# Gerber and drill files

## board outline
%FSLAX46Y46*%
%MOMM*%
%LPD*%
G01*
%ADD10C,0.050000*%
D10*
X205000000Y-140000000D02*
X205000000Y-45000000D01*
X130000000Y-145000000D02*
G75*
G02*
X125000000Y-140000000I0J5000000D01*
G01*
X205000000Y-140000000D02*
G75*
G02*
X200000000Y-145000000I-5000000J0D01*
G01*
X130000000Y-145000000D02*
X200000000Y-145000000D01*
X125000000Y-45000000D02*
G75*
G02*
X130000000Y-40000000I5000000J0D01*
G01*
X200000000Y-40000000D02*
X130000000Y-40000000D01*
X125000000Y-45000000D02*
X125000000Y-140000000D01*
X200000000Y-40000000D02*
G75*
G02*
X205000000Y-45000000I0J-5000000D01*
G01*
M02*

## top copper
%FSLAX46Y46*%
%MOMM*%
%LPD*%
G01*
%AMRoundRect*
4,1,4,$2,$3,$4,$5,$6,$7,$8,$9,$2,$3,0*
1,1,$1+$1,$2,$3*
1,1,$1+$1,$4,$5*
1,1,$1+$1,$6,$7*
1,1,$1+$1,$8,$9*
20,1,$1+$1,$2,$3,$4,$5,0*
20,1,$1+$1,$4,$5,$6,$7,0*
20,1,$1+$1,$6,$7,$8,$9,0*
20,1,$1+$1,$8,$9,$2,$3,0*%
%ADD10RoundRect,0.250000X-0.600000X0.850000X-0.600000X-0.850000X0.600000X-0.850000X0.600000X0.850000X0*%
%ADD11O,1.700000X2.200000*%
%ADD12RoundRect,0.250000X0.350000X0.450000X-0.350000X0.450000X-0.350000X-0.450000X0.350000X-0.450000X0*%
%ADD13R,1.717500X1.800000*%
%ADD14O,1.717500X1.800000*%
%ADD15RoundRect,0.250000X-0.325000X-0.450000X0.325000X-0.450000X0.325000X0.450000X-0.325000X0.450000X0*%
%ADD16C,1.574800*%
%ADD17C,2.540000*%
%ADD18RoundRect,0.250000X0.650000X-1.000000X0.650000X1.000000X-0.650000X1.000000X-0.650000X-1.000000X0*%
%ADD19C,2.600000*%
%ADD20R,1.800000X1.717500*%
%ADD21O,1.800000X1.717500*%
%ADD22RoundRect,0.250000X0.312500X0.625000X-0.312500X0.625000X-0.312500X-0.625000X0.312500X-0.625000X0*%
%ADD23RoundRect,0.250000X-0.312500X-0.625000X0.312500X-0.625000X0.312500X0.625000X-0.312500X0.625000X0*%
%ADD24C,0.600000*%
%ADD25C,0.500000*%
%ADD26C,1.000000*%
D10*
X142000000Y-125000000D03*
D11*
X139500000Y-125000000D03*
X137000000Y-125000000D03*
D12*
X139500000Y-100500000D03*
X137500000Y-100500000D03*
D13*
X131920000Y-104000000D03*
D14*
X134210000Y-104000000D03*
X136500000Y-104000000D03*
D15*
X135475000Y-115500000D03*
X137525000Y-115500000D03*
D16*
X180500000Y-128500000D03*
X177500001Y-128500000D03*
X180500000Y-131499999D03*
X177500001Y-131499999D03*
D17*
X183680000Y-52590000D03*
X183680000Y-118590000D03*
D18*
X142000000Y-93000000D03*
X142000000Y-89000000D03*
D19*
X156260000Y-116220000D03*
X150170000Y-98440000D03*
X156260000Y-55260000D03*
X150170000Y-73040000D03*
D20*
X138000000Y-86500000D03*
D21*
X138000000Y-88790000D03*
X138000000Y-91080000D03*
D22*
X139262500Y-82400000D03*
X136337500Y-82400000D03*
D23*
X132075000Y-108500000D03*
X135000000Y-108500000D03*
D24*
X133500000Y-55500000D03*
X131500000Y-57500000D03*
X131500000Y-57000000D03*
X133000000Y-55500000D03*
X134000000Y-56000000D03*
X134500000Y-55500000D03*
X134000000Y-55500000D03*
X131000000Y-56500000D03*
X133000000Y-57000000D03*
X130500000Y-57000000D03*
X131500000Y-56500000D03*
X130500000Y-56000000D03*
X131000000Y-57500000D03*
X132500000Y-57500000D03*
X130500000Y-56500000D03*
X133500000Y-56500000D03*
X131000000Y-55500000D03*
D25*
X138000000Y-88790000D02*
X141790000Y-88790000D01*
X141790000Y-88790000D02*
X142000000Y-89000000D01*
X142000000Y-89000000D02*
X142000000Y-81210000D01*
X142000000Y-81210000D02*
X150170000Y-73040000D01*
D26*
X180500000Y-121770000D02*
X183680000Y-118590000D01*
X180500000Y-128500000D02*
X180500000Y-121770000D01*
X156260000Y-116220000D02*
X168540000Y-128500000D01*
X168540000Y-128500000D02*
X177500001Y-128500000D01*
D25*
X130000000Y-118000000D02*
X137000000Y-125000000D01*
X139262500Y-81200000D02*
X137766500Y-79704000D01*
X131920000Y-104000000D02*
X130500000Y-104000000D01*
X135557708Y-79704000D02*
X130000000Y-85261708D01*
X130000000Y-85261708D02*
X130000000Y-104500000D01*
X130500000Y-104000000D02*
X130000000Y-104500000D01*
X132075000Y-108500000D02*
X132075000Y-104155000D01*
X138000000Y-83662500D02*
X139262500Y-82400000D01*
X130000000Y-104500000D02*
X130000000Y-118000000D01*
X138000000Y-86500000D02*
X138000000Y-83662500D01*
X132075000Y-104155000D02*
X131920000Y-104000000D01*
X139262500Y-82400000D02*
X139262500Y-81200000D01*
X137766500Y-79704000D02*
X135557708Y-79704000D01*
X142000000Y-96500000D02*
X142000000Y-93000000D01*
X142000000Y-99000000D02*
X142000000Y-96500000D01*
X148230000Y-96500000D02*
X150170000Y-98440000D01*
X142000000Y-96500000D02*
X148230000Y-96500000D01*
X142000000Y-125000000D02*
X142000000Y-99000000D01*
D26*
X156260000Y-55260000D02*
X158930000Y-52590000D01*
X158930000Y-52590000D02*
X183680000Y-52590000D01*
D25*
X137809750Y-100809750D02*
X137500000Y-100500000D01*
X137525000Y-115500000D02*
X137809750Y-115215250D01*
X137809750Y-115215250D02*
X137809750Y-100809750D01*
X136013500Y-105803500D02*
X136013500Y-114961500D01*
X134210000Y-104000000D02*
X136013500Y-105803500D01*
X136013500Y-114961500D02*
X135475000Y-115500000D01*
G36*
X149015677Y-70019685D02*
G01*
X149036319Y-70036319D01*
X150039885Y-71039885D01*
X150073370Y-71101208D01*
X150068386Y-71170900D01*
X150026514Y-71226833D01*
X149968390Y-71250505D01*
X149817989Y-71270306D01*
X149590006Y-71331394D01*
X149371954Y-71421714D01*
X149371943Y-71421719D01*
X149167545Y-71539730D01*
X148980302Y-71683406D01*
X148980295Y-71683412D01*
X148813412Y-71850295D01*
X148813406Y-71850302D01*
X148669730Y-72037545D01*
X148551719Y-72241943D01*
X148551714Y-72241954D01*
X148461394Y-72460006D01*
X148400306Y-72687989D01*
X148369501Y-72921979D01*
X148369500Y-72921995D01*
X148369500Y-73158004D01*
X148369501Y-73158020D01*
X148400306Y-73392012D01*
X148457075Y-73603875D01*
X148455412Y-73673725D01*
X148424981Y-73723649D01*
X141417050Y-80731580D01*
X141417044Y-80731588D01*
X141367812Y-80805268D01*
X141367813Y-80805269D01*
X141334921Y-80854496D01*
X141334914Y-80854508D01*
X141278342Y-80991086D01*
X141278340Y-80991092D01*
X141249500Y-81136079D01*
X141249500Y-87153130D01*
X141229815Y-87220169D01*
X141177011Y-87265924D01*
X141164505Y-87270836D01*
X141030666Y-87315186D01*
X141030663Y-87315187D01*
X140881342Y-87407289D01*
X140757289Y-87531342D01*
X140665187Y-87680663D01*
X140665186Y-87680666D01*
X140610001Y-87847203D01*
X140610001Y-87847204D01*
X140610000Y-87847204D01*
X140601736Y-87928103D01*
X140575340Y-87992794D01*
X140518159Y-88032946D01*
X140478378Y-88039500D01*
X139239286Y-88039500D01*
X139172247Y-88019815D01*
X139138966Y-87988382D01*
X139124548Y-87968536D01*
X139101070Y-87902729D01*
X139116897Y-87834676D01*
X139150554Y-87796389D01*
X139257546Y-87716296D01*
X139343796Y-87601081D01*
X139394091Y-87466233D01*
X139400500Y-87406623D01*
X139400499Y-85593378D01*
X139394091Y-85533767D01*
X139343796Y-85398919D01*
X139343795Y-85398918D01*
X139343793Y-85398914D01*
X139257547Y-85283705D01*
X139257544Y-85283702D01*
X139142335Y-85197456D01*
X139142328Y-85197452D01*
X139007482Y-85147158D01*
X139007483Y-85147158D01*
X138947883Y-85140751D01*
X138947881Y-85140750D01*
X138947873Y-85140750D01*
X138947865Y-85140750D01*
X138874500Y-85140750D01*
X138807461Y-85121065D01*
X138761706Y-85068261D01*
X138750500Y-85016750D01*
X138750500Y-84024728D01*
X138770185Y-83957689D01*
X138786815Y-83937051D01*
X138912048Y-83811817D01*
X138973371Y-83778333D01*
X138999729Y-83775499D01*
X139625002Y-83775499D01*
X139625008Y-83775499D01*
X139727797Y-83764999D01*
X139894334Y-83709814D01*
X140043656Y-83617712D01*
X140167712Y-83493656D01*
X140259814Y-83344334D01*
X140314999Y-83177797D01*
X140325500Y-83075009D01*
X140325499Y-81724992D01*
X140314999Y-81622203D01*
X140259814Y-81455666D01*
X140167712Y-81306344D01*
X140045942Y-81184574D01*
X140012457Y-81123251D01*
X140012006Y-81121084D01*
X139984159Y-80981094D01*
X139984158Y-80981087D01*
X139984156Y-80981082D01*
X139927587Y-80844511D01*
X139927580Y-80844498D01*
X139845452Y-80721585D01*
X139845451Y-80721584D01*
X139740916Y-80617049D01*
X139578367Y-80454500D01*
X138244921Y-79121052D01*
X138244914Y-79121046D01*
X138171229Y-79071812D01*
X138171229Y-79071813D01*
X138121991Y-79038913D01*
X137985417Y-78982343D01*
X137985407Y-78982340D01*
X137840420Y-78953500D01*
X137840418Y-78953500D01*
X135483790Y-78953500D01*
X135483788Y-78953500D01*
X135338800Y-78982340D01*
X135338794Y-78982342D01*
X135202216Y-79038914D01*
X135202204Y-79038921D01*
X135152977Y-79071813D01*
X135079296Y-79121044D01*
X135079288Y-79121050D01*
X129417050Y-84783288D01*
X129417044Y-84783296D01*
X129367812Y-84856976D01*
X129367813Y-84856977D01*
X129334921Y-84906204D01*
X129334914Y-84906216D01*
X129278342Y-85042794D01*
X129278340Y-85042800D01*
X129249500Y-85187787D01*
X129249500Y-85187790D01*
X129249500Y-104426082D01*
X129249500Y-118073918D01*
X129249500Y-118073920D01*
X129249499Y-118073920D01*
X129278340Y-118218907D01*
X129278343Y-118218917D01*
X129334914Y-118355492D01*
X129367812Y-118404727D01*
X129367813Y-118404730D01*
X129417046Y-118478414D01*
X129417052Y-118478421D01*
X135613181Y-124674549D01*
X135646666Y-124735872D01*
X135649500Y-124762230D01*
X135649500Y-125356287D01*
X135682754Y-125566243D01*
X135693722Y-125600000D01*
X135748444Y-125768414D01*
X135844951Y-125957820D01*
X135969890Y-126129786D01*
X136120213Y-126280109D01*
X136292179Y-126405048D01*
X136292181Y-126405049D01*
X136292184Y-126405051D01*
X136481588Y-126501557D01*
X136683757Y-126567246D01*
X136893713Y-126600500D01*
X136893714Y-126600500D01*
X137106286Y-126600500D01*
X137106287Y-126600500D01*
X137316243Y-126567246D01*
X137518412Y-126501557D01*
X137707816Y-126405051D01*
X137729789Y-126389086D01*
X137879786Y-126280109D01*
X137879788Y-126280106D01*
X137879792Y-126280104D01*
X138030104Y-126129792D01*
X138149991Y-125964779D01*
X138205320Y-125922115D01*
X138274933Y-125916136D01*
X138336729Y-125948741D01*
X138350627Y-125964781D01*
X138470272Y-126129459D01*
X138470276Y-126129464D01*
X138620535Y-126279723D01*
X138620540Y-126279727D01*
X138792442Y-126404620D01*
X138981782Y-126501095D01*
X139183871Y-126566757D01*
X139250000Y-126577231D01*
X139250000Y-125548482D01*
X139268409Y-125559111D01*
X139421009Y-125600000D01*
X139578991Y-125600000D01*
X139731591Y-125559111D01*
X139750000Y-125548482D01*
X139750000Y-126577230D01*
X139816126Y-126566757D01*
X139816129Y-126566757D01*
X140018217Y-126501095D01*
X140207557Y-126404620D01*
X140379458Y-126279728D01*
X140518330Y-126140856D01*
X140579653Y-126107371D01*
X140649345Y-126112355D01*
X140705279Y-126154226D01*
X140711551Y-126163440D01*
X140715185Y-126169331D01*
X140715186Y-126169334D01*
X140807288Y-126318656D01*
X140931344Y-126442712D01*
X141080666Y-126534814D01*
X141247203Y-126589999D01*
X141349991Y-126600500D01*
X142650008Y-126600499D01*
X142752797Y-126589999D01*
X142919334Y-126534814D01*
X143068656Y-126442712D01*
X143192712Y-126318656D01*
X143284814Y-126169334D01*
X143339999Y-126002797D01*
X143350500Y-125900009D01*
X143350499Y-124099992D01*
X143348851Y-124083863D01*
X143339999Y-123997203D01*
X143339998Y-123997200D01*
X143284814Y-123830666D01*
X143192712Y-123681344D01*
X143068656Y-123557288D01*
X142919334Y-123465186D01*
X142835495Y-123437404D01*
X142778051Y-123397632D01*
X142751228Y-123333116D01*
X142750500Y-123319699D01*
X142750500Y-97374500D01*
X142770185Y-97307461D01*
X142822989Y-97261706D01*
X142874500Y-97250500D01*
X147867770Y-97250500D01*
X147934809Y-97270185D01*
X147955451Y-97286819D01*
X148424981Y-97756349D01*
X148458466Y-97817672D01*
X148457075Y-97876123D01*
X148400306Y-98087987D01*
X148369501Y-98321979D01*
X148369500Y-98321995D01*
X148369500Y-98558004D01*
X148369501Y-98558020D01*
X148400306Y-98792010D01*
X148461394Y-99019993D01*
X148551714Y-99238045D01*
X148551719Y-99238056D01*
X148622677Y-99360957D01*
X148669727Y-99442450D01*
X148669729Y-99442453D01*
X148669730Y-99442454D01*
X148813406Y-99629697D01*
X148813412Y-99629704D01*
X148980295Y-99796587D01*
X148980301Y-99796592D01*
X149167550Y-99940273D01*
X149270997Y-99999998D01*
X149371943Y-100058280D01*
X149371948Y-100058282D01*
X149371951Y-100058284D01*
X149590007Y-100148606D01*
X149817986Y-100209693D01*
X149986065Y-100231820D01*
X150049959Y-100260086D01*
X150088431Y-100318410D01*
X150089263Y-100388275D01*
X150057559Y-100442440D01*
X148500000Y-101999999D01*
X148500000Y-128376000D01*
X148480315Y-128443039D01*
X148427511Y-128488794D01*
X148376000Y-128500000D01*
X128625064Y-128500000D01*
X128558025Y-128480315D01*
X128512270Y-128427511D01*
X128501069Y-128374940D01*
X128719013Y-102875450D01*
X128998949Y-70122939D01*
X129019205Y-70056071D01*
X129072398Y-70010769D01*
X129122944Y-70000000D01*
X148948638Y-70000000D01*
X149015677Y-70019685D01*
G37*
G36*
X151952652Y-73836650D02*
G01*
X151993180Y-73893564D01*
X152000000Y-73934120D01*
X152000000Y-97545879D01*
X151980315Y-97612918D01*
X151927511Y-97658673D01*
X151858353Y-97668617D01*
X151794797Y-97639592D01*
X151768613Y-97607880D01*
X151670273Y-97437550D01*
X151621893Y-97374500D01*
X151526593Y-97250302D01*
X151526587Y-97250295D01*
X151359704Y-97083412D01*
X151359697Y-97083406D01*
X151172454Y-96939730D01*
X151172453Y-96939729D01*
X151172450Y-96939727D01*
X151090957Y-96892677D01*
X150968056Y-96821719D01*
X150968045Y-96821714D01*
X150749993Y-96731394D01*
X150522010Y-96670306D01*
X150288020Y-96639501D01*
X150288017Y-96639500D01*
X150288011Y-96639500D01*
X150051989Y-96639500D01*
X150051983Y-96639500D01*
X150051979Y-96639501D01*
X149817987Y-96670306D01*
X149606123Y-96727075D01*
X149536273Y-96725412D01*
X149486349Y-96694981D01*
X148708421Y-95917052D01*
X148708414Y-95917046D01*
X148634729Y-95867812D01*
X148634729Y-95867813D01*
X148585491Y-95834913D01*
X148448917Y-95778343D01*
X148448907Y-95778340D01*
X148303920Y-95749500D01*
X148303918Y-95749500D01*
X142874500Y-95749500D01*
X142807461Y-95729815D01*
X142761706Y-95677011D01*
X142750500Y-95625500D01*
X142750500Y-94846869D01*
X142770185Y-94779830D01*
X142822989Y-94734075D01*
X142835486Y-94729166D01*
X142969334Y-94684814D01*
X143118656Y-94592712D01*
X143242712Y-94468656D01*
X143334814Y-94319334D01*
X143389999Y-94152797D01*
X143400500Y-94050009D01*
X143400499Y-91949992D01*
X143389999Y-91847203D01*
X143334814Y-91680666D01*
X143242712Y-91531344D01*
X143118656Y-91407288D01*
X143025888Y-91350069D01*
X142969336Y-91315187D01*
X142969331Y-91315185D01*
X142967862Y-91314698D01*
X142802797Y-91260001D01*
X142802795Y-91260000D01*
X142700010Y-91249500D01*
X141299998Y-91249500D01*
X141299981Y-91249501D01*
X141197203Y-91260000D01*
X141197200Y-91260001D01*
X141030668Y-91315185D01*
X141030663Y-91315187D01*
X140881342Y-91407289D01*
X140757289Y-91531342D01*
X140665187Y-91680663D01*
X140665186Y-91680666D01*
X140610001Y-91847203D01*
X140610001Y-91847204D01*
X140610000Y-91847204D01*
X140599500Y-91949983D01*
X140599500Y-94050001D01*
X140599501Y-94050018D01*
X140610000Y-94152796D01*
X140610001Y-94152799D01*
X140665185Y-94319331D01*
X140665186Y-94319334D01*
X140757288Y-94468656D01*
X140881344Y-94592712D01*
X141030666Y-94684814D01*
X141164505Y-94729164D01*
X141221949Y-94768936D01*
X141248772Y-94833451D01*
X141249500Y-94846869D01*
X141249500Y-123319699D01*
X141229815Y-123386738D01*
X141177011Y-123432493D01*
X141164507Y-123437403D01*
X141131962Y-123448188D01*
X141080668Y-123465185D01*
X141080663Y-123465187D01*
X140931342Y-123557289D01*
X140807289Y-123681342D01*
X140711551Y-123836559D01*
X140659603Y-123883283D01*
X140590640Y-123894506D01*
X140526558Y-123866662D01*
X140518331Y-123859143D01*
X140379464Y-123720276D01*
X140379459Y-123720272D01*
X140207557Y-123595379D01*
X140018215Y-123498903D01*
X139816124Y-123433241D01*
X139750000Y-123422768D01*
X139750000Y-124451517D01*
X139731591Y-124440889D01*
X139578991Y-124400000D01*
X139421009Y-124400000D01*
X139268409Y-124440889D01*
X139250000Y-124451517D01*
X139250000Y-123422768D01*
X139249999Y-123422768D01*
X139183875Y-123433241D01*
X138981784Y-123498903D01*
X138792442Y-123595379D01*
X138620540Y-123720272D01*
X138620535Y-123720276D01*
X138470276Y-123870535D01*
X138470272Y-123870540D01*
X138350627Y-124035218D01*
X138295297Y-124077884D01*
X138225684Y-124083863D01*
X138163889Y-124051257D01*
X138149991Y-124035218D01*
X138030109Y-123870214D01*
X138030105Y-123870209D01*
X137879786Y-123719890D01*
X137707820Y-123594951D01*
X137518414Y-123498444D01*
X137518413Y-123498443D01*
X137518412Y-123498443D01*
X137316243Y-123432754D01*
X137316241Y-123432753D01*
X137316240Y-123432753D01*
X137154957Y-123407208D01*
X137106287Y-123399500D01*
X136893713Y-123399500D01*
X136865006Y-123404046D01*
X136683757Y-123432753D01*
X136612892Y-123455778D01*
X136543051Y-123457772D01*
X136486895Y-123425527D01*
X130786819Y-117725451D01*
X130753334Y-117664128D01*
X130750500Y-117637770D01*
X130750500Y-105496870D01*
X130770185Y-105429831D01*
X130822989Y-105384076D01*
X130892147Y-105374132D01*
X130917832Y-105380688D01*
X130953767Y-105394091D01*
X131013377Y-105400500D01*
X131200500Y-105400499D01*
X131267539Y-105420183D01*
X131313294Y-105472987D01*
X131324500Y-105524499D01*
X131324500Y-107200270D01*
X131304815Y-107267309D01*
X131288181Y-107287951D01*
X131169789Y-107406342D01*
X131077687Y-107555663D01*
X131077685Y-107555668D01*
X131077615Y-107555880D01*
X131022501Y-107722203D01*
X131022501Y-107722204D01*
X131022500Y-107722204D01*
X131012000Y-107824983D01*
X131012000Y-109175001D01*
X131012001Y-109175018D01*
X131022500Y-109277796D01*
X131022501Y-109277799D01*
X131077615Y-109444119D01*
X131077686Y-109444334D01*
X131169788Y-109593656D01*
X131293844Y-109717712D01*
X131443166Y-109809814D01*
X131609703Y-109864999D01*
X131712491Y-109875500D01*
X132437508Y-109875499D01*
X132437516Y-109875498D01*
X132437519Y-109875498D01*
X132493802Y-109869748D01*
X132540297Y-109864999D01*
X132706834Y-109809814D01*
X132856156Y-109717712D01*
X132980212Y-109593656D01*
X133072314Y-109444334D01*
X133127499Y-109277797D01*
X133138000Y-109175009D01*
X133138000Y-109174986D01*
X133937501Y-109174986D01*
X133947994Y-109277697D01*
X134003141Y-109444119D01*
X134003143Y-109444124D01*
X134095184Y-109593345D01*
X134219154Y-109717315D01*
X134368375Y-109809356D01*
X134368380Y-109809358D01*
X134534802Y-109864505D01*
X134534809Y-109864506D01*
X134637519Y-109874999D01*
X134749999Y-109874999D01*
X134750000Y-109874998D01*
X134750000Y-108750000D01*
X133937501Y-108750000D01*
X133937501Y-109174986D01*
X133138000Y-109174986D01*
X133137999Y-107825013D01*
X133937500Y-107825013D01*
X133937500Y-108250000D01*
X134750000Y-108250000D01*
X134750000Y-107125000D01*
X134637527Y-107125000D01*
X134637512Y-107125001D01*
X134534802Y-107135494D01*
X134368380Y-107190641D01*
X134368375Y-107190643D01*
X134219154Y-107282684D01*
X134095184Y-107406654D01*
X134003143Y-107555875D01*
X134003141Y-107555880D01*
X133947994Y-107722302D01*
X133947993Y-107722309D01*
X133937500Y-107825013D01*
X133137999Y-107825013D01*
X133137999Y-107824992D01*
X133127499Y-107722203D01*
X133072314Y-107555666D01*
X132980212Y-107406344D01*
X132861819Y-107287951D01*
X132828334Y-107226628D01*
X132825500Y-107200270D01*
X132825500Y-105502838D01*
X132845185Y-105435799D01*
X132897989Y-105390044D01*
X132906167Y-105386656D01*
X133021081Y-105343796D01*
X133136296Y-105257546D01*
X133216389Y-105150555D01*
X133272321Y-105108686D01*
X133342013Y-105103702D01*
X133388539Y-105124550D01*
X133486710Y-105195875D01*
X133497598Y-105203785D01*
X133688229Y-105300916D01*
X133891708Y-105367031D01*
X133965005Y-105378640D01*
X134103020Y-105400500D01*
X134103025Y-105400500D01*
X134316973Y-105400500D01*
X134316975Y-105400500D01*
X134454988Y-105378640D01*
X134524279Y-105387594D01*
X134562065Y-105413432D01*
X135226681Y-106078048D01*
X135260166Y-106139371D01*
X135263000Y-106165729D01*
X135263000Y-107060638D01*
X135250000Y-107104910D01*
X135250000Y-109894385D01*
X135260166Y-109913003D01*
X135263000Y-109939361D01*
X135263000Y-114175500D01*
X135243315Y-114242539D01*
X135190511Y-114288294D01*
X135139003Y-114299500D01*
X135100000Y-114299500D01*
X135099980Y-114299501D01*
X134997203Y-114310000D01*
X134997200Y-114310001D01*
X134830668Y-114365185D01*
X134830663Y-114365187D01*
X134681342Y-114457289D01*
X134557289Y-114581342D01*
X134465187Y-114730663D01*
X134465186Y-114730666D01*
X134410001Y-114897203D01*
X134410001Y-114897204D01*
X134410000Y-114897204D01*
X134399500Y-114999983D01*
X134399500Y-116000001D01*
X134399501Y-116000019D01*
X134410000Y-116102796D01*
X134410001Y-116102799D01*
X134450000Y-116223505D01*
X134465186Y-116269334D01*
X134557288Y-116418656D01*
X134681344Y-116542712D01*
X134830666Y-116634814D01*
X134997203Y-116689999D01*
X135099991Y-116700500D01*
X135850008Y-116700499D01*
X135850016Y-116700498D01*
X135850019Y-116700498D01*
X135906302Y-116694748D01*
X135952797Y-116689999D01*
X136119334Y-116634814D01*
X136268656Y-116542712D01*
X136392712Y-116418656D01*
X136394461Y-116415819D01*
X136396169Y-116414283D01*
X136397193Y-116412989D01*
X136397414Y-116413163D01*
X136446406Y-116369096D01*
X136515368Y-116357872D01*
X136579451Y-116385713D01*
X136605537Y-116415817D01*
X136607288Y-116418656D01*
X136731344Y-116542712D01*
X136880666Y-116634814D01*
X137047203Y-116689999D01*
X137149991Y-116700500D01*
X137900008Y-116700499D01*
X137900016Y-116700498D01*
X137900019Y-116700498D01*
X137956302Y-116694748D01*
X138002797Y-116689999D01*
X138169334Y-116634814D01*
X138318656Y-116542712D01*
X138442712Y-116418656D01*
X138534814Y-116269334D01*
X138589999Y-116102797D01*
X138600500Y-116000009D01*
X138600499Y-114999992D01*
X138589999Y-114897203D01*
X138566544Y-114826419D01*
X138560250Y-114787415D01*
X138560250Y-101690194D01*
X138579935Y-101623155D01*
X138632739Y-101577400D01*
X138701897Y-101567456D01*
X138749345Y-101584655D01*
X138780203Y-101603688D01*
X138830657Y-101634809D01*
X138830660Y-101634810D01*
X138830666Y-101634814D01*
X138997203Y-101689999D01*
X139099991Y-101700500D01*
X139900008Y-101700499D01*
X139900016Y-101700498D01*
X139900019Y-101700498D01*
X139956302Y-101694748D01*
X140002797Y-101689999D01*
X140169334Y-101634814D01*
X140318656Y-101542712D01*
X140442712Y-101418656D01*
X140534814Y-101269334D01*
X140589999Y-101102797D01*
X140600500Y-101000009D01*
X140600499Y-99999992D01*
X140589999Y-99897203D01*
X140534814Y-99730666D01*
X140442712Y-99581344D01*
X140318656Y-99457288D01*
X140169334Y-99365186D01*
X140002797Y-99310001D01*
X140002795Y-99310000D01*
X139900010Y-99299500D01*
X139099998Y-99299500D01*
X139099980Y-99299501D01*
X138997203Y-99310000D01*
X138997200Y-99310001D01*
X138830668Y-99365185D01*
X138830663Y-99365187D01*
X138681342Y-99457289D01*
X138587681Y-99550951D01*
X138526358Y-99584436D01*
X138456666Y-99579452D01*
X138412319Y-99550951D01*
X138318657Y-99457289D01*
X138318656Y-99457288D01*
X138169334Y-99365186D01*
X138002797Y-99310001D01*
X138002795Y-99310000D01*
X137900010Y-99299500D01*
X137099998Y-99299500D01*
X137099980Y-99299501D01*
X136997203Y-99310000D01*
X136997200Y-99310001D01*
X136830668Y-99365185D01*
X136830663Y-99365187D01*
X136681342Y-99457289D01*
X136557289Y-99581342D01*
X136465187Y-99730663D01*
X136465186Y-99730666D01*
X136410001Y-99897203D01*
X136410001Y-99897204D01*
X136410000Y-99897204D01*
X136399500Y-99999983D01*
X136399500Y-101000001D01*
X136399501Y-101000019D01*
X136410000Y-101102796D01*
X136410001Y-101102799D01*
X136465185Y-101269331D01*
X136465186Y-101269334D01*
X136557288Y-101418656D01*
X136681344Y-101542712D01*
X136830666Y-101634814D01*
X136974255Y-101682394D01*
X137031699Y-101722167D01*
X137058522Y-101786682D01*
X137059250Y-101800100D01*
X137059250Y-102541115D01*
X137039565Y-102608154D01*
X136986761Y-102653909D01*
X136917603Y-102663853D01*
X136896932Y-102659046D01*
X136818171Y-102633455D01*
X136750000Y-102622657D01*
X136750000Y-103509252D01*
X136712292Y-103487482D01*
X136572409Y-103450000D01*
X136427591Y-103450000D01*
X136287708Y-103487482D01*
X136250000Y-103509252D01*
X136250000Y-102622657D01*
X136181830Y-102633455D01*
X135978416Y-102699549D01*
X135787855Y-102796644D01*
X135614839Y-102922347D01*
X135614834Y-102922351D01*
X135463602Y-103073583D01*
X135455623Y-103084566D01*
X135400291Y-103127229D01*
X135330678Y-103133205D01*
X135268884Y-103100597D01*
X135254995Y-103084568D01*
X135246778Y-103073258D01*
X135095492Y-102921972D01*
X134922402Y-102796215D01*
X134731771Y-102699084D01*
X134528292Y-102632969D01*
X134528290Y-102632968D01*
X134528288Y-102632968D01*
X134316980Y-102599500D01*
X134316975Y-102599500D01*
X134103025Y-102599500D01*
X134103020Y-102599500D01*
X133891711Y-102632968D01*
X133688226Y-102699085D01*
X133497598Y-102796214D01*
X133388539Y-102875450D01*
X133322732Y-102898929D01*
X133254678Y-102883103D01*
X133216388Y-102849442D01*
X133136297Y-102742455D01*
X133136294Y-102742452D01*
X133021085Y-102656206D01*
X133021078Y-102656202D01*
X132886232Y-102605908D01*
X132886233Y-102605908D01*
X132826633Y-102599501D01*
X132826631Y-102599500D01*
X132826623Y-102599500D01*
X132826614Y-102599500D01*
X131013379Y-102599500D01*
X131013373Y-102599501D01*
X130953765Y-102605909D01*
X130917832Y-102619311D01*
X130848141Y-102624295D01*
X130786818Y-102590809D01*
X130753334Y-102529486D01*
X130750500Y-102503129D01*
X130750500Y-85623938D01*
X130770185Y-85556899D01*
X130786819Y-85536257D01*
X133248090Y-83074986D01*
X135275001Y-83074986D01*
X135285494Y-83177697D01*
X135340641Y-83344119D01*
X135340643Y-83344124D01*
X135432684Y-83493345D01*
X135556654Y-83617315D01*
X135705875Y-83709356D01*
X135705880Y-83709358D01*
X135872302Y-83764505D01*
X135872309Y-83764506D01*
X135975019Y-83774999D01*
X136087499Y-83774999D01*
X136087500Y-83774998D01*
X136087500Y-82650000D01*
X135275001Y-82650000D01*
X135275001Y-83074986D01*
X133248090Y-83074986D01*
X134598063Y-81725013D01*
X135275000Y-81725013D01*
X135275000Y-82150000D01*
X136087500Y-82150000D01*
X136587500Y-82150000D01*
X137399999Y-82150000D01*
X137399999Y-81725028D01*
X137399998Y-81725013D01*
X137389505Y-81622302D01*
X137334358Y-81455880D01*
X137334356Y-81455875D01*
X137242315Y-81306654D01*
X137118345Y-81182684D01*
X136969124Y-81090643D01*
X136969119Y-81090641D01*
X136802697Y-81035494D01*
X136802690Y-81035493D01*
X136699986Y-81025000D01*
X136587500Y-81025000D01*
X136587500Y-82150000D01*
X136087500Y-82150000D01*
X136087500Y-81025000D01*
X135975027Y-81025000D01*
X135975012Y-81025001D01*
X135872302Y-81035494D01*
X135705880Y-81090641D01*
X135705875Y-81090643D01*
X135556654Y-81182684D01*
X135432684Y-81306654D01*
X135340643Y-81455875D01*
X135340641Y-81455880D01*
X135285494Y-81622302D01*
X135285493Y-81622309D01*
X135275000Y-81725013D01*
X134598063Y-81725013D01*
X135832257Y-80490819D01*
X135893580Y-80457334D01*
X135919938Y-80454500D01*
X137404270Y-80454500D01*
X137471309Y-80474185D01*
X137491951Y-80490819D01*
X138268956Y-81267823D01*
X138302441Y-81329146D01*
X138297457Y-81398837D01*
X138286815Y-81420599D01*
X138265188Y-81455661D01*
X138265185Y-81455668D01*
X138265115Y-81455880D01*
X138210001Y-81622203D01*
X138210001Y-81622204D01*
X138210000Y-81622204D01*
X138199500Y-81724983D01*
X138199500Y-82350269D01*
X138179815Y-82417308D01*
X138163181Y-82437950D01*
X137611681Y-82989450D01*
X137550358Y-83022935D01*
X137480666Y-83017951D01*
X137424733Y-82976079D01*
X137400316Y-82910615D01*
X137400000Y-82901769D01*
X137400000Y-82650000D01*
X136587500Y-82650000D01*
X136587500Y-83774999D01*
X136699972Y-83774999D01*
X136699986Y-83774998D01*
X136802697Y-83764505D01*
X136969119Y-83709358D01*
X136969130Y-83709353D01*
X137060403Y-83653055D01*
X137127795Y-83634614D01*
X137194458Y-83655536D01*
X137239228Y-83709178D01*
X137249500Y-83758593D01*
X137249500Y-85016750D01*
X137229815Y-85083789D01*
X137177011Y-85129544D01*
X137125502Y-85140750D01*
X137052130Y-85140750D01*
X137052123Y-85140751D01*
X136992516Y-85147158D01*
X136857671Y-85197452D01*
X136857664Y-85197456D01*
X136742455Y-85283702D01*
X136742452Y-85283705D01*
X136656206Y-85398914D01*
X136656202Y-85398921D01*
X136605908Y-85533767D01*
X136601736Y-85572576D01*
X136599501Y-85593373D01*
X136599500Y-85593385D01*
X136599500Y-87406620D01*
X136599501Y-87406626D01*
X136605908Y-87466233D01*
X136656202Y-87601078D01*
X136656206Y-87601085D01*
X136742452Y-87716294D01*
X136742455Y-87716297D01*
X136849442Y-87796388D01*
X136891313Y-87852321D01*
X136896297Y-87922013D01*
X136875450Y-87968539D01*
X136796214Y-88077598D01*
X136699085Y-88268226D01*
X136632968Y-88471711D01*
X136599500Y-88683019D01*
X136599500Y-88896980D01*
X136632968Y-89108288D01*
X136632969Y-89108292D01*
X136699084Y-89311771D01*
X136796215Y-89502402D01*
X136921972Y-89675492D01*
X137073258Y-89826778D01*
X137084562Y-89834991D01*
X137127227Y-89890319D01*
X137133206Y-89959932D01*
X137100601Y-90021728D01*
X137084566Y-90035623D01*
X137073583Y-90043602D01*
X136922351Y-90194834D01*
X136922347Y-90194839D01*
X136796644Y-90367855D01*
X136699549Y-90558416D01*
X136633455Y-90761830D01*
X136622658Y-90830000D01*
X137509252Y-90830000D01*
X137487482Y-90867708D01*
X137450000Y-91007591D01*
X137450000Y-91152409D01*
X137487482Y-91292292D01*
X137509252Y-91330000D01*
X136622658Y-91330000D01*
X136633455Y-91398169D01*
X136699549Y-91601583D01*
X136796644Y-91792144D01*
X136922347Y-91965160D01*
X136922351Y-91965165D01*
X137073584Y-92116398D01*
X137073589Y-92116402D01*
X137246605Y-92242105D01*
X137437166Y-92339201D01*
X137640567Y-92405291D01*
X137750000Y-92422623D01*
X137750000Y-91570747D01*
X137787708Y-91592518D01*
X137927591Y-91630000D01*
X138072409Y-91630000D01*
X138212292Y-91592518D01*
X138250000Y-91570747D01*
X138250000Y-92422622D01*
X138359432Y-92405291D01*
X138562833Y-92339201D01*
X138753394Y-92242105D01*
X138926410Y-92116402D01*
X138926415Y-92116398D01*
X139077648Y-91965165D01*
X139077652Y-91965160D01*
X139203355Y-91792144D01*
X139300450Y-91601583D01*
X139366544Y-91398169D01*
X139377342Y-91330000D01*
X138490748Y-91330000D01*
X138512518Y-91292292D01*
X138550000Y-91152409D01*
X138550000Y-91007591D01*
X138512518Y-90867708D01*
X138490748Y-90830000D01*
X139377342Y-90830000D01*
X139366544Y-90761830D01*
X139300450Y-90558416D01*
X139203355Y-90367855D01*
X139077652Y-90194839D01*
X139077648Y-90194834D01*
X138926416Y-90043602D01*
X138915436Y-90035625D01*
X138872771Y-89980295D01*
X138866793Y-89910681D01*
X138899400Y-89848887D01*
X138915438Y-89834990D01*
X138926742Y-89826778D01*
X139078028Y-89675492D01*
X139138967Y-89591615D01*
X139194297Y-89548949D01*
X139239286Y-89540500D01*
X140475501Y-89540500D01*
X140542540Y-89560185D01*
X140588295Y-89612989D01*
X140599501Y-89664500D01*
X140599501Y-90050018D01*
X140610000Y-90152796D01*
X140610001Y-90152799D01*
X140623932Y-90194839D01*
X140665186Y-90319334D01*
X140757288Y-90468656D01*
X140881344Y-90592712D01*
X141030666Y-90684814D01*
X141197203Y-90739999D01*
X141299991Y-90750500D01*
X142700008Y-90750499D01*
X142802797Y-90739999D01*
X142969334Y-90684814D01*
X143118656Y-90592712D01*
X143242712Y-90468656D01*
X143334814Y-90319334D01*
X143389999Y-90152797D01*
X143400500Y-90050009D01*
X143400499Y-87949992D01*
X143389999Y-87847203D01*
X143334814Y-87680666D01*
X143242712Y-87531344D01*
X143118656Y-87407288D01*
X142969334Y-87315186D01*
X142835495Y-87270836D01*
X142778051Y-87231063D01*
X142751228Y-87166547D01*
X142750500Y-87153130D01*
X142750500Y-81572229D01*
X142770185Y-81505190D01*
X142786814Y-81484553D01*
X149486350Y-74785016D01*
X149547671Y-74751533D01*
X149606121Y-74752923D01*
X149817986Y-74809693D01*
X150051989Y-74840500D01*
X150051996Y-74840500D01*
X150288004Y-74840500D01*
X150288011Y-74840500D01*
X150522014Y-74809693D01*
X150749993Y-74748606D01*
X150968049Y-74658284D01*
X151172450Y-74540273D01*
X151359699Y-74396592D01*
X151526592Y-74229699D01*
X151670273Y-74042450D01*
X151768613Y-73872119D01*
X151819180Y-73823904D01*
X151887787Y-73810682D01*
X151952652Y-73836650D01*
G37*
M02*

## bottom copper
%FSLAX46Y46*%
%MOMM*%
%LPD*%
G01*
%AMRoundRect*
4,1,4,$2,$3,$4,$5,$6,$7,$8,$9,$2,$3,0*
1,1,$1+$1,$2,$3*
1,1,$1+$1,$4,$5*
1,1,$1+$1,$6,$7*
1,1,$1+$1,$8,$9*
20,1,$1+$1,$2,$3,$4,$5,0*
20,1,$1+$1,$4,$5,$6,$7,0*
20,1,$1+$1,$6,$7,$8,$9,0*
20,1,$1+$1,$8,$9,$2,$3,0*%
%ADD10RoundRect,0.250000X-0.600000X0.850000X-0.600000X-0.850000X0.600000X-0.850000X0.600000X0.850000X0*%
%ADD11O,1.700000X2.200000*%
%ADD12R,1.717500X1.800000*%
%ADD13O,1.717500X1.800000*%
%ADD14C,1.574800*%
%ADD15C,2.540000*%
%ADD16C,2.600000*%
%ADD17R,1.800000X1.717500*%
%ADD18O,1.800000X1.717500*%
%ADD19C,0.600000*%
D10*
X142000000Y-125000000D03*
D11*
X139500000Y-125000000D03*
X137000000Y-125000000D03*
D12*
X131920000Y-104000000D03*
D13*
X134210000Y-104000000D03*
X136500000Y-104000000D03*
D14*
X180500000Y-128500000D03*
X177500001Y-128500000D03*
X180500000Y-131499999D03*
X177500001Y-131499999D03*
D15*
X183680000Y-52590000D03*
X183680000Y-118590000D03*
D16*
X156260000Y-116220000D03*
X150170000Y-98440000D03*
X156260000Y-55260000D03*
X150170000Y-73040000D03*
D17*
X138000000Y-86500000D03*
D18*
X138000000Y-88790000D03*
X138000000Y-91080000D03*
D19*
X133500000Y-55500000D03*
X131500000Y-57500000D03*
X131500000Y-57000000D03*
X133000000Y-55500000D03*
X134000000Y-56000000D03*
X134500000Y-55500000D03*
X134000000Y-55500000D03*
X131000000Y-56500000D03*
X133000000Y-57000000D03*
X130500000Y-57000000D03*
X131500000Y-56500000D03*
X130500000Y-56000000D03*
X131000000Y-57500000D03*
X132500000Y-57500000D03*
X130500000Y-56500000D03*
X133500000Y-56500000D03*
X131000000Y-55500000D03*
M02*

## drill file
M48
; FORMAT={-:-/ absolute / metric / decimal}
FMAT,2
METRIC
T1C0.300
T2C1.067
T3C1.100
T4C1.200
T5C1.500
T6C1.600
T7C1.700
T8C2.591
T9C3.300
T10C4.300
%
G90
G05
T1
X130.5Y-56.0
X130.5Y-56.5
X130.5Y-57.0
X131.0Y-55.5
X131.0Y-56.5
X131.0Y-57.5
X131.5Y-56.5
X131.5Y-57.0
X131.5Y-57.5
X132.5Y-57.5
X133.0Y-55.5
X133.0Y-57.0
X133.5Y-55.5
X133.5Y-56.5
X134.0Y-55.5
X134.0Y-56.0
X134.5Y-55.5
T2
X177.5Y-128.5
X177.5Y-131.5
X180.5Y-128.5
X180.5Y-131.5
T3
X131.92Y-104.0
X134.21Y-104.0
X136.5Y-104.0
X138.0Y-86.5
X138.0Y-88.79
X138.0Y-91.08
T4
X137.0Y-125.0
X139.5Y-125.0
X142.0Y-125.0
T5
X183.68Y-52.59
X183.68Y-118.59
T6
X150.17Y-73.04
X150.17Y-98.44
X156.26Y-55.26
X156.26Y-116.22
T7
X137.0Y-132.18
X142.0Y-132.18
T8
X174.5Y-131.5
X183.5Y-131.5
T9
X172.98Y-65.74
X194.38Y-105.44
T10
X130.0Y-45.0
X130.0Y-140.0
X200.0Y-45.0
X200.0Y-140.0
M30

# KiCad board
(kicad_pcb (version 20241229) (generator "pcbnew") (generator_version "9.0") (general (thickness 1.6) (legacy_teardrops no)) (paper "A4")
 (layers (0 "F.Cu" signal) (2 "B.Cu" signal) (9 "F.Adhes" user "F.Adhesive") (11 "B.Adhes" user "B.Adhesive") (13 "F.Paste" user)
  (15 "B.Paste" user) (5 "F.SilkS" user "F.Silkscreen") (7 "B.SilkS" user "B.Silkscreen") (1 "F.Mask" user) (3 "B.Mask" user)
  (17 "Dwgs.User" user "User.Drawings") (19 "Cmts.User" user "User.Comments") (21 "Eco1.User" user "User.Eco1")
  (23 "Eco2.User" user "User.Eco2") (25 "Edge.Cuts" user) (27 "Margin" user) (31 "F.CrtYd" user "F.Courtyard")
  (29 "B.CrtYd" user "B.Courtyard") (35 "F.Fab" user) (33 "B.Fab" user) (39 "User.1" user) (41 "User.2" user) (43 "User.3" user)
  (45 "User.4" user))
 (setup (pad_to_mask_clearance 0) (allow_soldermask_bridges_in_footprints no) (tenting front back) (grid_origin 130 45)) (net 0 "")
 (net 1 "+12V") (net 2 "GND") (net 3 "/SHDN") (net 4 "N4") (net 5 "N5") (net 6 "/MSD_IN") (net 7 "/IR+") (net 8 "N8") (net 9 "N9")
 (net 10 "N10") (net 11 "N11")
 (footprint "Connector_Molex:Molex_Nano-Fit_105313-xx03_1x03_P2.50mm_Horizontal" (layer "F.Cu") (at 142 125 -90)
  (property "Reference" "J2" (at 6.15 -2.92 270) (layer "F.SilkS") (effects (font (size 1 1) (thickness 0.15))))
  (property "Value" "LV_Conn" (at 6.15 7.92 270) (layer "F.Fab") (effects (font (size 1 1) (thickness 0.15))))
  (pad "" np_thru_hole circle (at 7.18 0 270) (size 1.7 1.7) (drill 1.7) (layers "*.Cu" "*.Mask"))
  (pad "" np_thru_hole circle (at 7.18 5 270) (size 1.7 1.7) (drill 1.7) (layers "*.Cu" "*.Mask"))
  (pad "1" thru_hole roundrect (at 0 0 270) (size 2.2 1.7) (drill 1.2) (layers "*.Cu" "*.Mask") (remove_unused_layers no)
   (roundrect_rratio 0.147059) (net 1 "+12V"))
  (pad "2" thru_hole oval (at 0 2.5 270) (size 2.2 1.7) (drill 1.2) (layers "*.Cu" "*.Mask") (remove_unused_layers no) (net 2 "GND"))
  (pad "3" thru_hole oval (at 0 5 270) (size 2.2 1.7) (drill 1.2) (layers "*.Cu" "*.Mask") (remove_unused_layers no) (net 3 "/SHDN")))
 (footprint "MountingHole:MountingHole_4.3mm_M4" (layer "F.Cu") (at 130 140)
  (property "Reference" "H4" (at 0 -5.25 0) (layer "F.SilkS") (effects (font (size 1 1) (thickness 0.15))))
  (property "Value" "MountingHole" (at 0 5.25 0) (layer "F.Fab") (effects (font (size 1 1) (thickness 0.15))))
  (pad "" np_thru_hole circle (at 0 0) (size 4.3 4.3) (drill 4.3) (layers "*.Cu" "*.Mask")))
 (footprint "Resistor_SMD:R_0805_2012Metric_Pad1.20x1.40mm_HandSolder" (layer "F.Cu") (at 138.5 100.5 180)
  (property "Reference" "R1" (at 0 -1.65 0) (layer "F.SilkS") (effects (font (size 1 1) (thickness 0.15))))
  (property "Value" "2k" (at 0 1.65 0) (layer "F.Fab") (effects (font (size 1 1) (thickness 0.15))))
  (pad "1" smd roundrect (at -1 0 180) (size 1.2 1.4) (layers "F.Cu" "F.Mask" "F.Paste") (roundrect_rratio 0.208333) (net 1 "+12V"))
  (pad "2" smd roundrect (at 1 0 180) (size 1.2 1.4) (layers "F.Cu" "F.Mask" "F.Paste") (roundrect_rratio 0.208333) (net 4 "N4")))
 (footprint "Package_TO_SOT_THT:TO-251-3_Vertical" (layer "F.Cu") (at 131.92 104)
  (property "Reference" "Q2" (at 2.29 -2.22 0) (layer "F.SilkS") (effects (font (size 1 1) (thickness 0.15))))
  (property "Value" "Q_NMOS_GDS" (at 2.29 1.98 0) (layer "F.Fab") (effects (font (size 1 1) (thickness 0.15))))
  (pad "1" thru_hole rect (at 0 0) (size 1.7175 1.8) (drill 1.1) (layers "*.Cu" "*.Mask") (remove_unused_layers no) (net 3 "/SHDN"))
  (pad "2" thru_hole oval (at 2.29 0) (size 1.7175 1.8) (drill 1.1) (layers "*.Cu" "*.Mask") (remove_unused_layers no) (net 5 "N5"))
  (pad "3" thru_hole oval (at 4.58 0) (size 1.7175 1.8) (drill 1.1) (layers "*.Cu" "*.Mask") (remove_unused_layers no) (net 2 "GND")))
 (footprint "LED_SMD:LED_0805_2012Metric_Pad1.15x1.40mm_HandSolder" (layer "F.Cu") (at 136.5 115.5)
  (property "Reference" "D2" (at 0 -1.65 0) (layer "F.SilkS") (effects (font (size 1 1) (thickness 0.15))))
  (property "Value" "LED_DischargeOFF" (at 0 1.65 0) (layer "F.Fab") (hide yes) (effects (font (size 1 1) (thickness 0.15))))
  (pad "1" smd roundrect (at -1.025 0) (size 1.15 1.4) (layers "F.Cu" "F.Mask" "F.Paste") (roundrect_rratio 0.217391) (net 5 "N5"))
  (pad "2" smd roundrect (at 1.025 0) (size 1.15 1.4) (layers "F.Cu" "F.Mask" "F.Paste") (roundrect_rratio 0.217391) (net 4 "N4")))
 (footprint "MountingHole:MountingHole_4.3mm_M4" (layer "F.Cu") (at 130 45)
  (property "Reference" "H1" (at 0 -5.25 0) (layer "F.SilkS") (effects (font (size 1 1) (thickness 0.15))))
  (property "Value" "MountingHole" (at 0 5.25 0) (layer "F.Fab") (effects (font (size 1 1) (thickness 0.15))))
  (pad "" np_thru_hole circle (at 0 0) (size 4.3 4.3) (drill 4.3) (layers "*.Cu" "*.Mask")))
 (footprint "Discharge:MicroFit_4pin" (layer "F.Cu") (at 179.2484 130.0186 180)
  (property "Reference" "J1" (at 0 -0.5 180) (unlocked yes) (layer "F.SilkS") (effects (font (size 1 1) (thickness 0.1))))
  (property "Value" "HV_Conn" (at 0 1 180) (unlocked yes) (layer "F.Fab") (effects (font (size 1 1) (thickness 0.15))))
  (pad "" np_thru_hole circle (at -4.251599 -1.481399 180) (size 2.5908 2.5908) (drill 2.5908) (layers))
  (pad "" np_thru_hole circle (at 4.748398 -1.481399 180) (size 2.5908 2.5908) (drill 2.5908) (layers))
  (pad "1" thru_hole circle (at -1.2516 1.5186 180) (size 1.5748 1.5748) (drill 1.0668) (layers "*.Cu" "*.Mask") (remove_unused_layers no)
   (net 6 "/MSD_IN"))
  (pad "2" thru_hole circle (at 1.748399 1.5186 180) (size 1.5748 1.5748) (drill 1.0668) (layers "*.Cu" "*.Mask") (remove_unused_layers no)
   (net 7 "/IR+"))
  (pad "3" thru_hole circle (at -1.2516 -1.481399 180) (size 1.5748 1.5748) (drill 1.0668) (layers "*.Cu" "*.Mask")
   (remove_unused_layers no) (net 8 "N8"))
  (pad "4" thru_hole circle (at 1.748399 -1.481399 180) (size 1.5748 1.5748) (drill 1.0668) (layers "*.Cu" "*.Mask")
   (remove_unused_layers no) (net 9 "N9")))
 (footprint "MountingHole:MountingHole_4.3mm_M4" (layer "F.Cu") (at 200 140)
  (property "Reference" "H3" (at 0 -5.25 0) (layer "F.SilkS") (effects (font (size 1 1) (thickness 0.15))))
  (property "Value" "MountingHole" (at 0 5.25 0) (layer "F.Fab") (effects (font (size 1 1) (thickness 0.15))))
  (pad "" np_thru_hole circle (at 0 0) (size 4.3 4.3) (drill 4.3) (layers "*.Cu" "*.Mask")))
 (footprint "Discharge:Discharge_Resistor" (layer "F.Cu") (at 183.68 85.59 -90)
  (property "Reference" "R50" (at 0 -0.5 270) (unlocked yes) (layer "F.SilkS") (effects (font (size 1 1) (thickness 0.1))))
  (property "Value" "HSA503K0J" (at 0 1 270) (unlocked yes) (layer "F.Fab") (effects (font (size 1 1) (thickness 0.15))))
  (pad "" np_thru_hole circle (at -19.85 10.7 270) (size 3.3 3.3) (drill 3.3) (layers "*.Cu" "*.Mask"))
  (pad "" np_thru_hole circle (at 19.85 -10.7 270) (size 3.3 3.3) (drill 3.3) (layers "*.Cu" "*.Mask"))
  (pad "1" thru_hole circle (at -33 0 270) (size 2.54 2.54) (drill 1.5) (layers "*.Cu" "*.Mask") (remove_unused_layers no) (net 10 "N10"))
  (pad "2" thru_hole circle (at 33 0 270) (size 2.54 2.54) (drill 1.5) (layers "*.Cu" "*.Mask") (remove_unused_layers no) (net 6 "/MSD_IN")))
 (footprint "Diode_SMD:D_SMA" (layer "F.Cu") (at 142 91 90)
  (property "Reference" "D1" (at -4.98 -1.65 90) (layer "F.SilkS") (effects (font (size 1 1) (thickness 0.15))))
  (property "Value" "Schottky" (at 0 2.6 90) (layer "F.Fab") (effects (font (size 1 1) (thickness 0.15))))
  (pad "1" smd roundrect (at -2 0 90) (size 2.5 1.8) (layers "F.Cu" "F.Mask" "F.Paste") (roundrect_rratio 0.1388888889) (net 1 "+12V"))
  (pad "2" smd roundrect (at 2 0 90) (size 2.5 1.8) (layers "F.Cu" "F.Mask" "F.Paste") (roundrect_rratio 0.1388888889) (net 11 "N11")))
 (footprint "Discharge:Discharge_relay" (layer "F.Cu") (at 154.555 85.74 -90)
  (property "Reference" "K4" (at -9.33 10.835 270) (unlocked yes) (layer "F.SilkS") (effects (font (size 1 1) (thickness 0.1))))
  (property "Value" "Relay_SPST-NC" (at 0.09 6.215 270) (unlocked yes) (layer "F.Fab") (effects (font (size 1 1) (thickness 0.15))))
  (pad "1" thru_hole circle (at 30.48 -1.705 90) (size 2.6 2.6) (drill 1.6) (layers "*.Cu" "*.Mask") (remove_unused_layers no)
   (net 7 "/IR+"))
  (pad "2" thru_hole circle (at 12.7 4.385 90) (size 2.6 2.6) (drill 1.6) (layers "*.Cu" "*.Mask") (remove_unused_layers no) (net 1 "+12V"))
  (pad "4" thru_hole circle (at -30.48 -1.705 90) (size 2.6 2.6) (drill 1.6) (layers "*.Cu" "*.Mask") (remove_unused_layers no)
   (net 10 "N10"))
  (pad "5" thru_hole circle (at -12.7 4.385 90) (size 2.6 2.6) (drill 1.6) (layers "*.Cu" "*.Mask") (remove_unused_layers no) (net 11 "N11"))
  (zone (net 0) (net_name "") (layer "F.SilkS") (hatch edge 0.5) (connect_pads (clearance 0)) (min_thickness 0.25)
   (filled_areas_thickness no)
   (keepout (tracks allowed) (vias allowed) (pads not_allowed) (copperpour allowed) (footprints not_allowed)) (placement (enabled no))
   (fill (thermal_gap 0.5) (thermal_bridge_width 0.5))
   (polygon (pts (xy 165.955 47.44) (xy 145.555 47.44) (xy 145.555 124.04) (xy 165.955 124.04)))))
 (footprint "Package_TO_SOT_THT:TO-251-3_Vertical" (layer "F.Cu") (at 138 86.5 -90)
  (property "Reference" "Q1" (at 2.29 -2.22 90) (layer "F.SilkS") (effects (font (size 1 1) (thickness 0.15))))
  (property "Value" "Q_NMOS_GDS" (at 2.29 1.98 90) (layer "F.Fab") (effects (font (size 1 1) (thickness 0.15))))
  (pad "1" thru_hole rect (at 0 0 270) (size 1.7175 1.8) (drill 1.1) (layers "*.Cu" "*.Mask") (remove_unused_layers no) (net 3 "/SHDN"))
  (pad "2" thru_hole oval (at 2.29 0 270) (size 1.7175 1.8) (drill 1.1) (layers "*.Cu" "*.Mask") (remove_unused_layers no) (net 11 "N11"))
  (pad "3" thru_hole oval (at 4.58 0 270) (size 1.7175 1.8) (drill 1.1) (layers "*.Cu" "*.Mask") (remove_unused_layers no) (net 2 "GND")))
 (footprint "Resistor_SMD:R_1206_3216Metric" (layer "F.Cu") (at 137.8 82.4 180)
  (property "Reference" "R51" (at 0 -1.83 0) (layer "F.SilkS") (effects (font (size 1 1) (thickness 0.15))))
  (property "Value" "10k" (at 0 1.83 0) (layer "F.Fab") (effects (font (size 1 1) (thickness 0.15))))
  (pad "1" smd roundrect (at -1.4625 0 180) (size 1.125 1.75) (layers "F.Cu" "F.Mask" "F.Paste") (roundrect_rratio 0.222222) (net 3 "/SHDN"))
  (pad "2" smd roundrect (at 1.4625 0 180) (size 1.125 1.75) (layers "F.Cu" "F.Mask" "F.Paste") (roundrect_rratio 0.222222) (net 2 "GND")))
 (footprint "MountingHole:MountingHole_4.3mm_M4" (layer "F.Cu") (at 200 45)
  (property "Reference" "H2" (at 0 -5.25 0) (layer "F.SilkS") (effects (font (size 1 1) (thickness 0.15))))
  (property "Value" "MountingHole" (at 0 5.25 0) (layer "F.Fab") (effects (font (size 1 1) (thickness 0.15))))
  (pad "" np_thru_hole circle (at 0 0) (size 4.3 4.3) (drill 4.3) (layers "*.Cu" "*.Mask")))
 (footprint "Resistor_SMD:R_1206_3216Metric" (layer "F.Cu") (at 133.5375 108.5)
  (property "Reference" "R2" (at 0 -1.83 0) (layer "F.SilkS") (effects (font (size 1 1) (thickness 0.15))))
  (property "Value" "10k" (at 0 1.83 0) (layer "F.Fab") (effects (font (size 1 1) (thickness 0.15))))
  (pad "1" smd roundrect (at -1.4625 0) (size 1.125 1.75) (layers "F.Cu" "F.Mask" "F.Paste") (roundrect_rratio 0.222222) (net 3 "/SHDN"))
  (pad "2" smd roundrect (at 1.4625 0) (size 1.125 1.75) (layers "F.Cu" "F.Mask" "F.Paste") (roundrect_rratio 0.222222) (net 2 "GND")))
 (gr_line (start 205 140) (end 205 45) (stroke (width 0.05) (type default)) (layer "Edge.Cuts"))
 (gr_arc (start 130 145) (mid 126.464466 143.535534) (end 125 140) (stroke (width 0.05) (type default)) (layer "Edge.Cuts"))
 (gr_arc (start 205 140) (mid 203.535534 143.535534) (end 200 145) (stroke (width 0.05) (type default)) (layer "Edge.Cuts"))
 (gr_line (start 130 145) (end 200 145) (stroke (width 0.05) (type default)) (layer "Edge.Cuts"))
 (gr_arc (start 125 45) (mid 126.464466 41.464466) (end 130 40) (stroke (width 0.05) (type default)) (layer "Edge.Cuts"))
 (gr_line (start 200 40) (end 130 40) (stroke (width 0.05) (type default)) (layer "Edge.Cuts"))
 (gr_line (start 125 45) (end 125 140) (stroke (width 0.05) (type default)) (layer "Edge.Cuts"))
 (gr_arc (start 200 40) (mid 203.535534 41.464466) (end 205 45) (stroke (width 0.05) (type default)) (layer "Edge.Cuts"))
 (via (at 133.5 55.5) (size 0.6) (drill 0.3) (layers "F.Cu" "B.Cu") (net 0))
 (via (at 131.5 57.5) (size 0.6) (drill 0.3) (layers "F.Cu" "B.Cu") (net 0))
 (via (at 131.5 57) (size 0.6) (drill 0.3) (layers "F.Cu" "B.Cu") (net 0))
 (via (at 133 55.5) (size 0.6) (drill 0.3) (layers "F.Cu" "B.Cu") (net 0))
 (via (at 134 56) (size 0.6) (drill 0.3) (layers "F.Cu" "B.Cu") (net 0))
 (via (at 134.5 55.5) (size 0.6) (drill 0.3) (layers "F.Cu" "B.Cu") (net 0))
 (via (at 134 55.5) (size 0.6) (drill 0.3) (layers "F.Cu" "B.Cu") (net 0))
 (via (at 131 56.5) (size 0.6) (drill 0.3) (layers "F.Cu" "B.Cu") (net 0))
 (via (at 133 57) (size 0.6) (drill 0.3) (layers "F.Cu" "B.Cu") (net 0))
 (via (at 130.5 57) (size 0.6) (drill 0.3) (layers "F.Cu" "B.Cu") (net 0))
 (via (at 131.5 56.5) (size 0.6) (drill 0.3) (layers "F.Cu" "B.Cu") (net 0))
 (via (at 130.5 56) (size 0.6) (drill 0.3) (layers "F.Cu" "B.Cu") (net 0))
 (via (at 131 57.5) (size 0.6) (drill 0.3) (layers "F.Cu" "B.Cu") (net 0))
 (via (at 132.5 57.5) (size 0.6) (drill 0.3) (layers "F.Cu" "B.Cu") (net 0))
 (via (at 130.5 56.5) (size 0.6) (drill 0.3) (layers "F.Cu" "B.Cu") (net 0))
 (via (at 133.5 56.5) (size 0.6) (drill 0.3) (layers "F.Cu" "B.Cu") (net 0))
 (via (at 131 55.5) (size 0.6) (drill 0.3) (layers "F.Cu" "B.Cu") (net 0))
 (segment (start 138 88.79) (end 141.79 88.79) (width 0.5) (layer "F.Cu") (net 11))
 (segment (start 141.79 88.79) (end 142 89) (width 0.5) (layer "F.Cu") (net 11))
 (segment (start 142 89) (end 142 81.21) (width 0.5) (layer "F.Cu") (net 11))
 (segment (start 142 81.21) (end 150.17 73.04) (width 0.5) (layer "F.Cu") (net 11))
 (segment (start 180.5 121.77) (end 183.68 118.59) (width 1) (layer "F.Cu") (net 6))
 (segment (start 180.5 128.5) (end 180.5 121.77) (width 1) (layer "F.Cu") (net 6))
 (segment (start 156.26 116.22) (end 168.54 128.5) (width 1) (layer "F.Cu") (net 7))
 (segment (start 168.54 128.5) (end 177.500001 128.5) (width 1) (layer "F.Cu") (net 7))
 (segment (start 130 118) (end 137 125) (width 0.5) (layer "F.Cu") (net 3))
 (segment (start 139.2625 81.2) (end 137.7665 79.704) (width 0.5) (layer "F.Cu") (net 3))
 (segment (start 131.92 104) (end 130.5 104) (width 0.5) (layer "F.Cu") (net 3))
 (segment (start 135.557708 79.704) (end 130 85.261708) (width 0.5) (layer "F.Cu") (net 3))
 (segment (start 130 85.261708) (end 130 104.5) (width 0.5) (layer "F.Cu") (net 3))
 (segment (start 130.5 104) (end 130 104.5) (width 0.5) (layer "F.Cu") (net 3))
 (segment (start 132.075 108.5) (end 132.075 104.155) (width 0.5) (layer "F.Cu") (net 3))
 (segment (start 138 83.6625) (end 139.2625 82.4) (width 0.5) (layer "F.Cu") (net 3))
 (segment (start 130 104.5) (end 130 118) (width 0.5) (layer "F.Cu") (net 3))
 (segment (start 138 86.5) (end 138 83.6625) (width 0.5) (layer "F.Cu") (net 3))
 (segment (start 132.075 104.155) (end 131.92 104) (width 0.5) (layer "F.Cu") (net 3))
 (segment (start 139.2625 82.4) (end 139.2625 81.2) (width 0.5) (layer "F.Cu") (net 3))
 (segment (start 137.7665 79.704) (end 135.557708 79.704) (width 0.5) (layer "F.Cu") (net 3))
 (segment (start 142 96.5) (end 142 93) (width 0.5) (layer "F.Cu") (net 1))
 (segment (start 142 99) (end 142 96.5) (width 0.5) (layer "F.Cu") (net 1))
 (segment (start 148.23 96.5) (end 150.17 98.44) (width 0.5) (layer "F.Cu") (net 1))
 (segment (start 142 96.5) (end 148.23 96.5) (width 0.5) (layer "F.Cu") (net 1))
 (segment (start 142 125) (end 142 99) (width 0.5) (layer "F.Cu") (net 1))
 (segment (start 156.26 55.26) (end 158.93 52.59) (width 1) (layer "F.Cu") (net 10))
 (segment (start 158.93 52.59) (end 183.68 52.59) (width 1) (layer "F.Cu") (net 10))
 (segment (start 137.80975 100.80975) (end 137.5 100.5) (width 0.5) (layer "F.Cu") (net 4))
 (segment (start 137.525 115.5) (end 137.80975 115.21525) (width 0.5) (layer "F.Cu") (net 4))
 (segment (start 137.80975 115.21525) (end 137.80975 100.80975) (width 0.5) (layer "F.Cu") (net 4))
 (segment (start 136.0135 105.8035) (end 136.0135 114.9615) (width 0.5) (layer "F.Cu") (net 5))
 (segment (start 134.21 104) (end 136.0135 105.8035) (width 0.5) (layer "F.Cu") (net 5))
 (segment (start 136.0135 114.9615) (end 135.475 115.5) (width 0.5) (layer "F.Cu") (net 5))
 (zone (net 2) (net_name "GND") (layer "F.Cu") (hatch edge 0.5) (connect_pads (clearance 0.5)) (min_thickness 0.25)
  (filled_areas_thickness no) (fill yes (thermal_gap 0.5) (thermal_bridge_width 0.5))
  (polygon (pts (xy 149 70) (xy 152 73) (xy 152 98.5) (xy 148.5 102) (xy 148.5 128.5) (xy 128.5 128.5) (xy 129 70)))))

